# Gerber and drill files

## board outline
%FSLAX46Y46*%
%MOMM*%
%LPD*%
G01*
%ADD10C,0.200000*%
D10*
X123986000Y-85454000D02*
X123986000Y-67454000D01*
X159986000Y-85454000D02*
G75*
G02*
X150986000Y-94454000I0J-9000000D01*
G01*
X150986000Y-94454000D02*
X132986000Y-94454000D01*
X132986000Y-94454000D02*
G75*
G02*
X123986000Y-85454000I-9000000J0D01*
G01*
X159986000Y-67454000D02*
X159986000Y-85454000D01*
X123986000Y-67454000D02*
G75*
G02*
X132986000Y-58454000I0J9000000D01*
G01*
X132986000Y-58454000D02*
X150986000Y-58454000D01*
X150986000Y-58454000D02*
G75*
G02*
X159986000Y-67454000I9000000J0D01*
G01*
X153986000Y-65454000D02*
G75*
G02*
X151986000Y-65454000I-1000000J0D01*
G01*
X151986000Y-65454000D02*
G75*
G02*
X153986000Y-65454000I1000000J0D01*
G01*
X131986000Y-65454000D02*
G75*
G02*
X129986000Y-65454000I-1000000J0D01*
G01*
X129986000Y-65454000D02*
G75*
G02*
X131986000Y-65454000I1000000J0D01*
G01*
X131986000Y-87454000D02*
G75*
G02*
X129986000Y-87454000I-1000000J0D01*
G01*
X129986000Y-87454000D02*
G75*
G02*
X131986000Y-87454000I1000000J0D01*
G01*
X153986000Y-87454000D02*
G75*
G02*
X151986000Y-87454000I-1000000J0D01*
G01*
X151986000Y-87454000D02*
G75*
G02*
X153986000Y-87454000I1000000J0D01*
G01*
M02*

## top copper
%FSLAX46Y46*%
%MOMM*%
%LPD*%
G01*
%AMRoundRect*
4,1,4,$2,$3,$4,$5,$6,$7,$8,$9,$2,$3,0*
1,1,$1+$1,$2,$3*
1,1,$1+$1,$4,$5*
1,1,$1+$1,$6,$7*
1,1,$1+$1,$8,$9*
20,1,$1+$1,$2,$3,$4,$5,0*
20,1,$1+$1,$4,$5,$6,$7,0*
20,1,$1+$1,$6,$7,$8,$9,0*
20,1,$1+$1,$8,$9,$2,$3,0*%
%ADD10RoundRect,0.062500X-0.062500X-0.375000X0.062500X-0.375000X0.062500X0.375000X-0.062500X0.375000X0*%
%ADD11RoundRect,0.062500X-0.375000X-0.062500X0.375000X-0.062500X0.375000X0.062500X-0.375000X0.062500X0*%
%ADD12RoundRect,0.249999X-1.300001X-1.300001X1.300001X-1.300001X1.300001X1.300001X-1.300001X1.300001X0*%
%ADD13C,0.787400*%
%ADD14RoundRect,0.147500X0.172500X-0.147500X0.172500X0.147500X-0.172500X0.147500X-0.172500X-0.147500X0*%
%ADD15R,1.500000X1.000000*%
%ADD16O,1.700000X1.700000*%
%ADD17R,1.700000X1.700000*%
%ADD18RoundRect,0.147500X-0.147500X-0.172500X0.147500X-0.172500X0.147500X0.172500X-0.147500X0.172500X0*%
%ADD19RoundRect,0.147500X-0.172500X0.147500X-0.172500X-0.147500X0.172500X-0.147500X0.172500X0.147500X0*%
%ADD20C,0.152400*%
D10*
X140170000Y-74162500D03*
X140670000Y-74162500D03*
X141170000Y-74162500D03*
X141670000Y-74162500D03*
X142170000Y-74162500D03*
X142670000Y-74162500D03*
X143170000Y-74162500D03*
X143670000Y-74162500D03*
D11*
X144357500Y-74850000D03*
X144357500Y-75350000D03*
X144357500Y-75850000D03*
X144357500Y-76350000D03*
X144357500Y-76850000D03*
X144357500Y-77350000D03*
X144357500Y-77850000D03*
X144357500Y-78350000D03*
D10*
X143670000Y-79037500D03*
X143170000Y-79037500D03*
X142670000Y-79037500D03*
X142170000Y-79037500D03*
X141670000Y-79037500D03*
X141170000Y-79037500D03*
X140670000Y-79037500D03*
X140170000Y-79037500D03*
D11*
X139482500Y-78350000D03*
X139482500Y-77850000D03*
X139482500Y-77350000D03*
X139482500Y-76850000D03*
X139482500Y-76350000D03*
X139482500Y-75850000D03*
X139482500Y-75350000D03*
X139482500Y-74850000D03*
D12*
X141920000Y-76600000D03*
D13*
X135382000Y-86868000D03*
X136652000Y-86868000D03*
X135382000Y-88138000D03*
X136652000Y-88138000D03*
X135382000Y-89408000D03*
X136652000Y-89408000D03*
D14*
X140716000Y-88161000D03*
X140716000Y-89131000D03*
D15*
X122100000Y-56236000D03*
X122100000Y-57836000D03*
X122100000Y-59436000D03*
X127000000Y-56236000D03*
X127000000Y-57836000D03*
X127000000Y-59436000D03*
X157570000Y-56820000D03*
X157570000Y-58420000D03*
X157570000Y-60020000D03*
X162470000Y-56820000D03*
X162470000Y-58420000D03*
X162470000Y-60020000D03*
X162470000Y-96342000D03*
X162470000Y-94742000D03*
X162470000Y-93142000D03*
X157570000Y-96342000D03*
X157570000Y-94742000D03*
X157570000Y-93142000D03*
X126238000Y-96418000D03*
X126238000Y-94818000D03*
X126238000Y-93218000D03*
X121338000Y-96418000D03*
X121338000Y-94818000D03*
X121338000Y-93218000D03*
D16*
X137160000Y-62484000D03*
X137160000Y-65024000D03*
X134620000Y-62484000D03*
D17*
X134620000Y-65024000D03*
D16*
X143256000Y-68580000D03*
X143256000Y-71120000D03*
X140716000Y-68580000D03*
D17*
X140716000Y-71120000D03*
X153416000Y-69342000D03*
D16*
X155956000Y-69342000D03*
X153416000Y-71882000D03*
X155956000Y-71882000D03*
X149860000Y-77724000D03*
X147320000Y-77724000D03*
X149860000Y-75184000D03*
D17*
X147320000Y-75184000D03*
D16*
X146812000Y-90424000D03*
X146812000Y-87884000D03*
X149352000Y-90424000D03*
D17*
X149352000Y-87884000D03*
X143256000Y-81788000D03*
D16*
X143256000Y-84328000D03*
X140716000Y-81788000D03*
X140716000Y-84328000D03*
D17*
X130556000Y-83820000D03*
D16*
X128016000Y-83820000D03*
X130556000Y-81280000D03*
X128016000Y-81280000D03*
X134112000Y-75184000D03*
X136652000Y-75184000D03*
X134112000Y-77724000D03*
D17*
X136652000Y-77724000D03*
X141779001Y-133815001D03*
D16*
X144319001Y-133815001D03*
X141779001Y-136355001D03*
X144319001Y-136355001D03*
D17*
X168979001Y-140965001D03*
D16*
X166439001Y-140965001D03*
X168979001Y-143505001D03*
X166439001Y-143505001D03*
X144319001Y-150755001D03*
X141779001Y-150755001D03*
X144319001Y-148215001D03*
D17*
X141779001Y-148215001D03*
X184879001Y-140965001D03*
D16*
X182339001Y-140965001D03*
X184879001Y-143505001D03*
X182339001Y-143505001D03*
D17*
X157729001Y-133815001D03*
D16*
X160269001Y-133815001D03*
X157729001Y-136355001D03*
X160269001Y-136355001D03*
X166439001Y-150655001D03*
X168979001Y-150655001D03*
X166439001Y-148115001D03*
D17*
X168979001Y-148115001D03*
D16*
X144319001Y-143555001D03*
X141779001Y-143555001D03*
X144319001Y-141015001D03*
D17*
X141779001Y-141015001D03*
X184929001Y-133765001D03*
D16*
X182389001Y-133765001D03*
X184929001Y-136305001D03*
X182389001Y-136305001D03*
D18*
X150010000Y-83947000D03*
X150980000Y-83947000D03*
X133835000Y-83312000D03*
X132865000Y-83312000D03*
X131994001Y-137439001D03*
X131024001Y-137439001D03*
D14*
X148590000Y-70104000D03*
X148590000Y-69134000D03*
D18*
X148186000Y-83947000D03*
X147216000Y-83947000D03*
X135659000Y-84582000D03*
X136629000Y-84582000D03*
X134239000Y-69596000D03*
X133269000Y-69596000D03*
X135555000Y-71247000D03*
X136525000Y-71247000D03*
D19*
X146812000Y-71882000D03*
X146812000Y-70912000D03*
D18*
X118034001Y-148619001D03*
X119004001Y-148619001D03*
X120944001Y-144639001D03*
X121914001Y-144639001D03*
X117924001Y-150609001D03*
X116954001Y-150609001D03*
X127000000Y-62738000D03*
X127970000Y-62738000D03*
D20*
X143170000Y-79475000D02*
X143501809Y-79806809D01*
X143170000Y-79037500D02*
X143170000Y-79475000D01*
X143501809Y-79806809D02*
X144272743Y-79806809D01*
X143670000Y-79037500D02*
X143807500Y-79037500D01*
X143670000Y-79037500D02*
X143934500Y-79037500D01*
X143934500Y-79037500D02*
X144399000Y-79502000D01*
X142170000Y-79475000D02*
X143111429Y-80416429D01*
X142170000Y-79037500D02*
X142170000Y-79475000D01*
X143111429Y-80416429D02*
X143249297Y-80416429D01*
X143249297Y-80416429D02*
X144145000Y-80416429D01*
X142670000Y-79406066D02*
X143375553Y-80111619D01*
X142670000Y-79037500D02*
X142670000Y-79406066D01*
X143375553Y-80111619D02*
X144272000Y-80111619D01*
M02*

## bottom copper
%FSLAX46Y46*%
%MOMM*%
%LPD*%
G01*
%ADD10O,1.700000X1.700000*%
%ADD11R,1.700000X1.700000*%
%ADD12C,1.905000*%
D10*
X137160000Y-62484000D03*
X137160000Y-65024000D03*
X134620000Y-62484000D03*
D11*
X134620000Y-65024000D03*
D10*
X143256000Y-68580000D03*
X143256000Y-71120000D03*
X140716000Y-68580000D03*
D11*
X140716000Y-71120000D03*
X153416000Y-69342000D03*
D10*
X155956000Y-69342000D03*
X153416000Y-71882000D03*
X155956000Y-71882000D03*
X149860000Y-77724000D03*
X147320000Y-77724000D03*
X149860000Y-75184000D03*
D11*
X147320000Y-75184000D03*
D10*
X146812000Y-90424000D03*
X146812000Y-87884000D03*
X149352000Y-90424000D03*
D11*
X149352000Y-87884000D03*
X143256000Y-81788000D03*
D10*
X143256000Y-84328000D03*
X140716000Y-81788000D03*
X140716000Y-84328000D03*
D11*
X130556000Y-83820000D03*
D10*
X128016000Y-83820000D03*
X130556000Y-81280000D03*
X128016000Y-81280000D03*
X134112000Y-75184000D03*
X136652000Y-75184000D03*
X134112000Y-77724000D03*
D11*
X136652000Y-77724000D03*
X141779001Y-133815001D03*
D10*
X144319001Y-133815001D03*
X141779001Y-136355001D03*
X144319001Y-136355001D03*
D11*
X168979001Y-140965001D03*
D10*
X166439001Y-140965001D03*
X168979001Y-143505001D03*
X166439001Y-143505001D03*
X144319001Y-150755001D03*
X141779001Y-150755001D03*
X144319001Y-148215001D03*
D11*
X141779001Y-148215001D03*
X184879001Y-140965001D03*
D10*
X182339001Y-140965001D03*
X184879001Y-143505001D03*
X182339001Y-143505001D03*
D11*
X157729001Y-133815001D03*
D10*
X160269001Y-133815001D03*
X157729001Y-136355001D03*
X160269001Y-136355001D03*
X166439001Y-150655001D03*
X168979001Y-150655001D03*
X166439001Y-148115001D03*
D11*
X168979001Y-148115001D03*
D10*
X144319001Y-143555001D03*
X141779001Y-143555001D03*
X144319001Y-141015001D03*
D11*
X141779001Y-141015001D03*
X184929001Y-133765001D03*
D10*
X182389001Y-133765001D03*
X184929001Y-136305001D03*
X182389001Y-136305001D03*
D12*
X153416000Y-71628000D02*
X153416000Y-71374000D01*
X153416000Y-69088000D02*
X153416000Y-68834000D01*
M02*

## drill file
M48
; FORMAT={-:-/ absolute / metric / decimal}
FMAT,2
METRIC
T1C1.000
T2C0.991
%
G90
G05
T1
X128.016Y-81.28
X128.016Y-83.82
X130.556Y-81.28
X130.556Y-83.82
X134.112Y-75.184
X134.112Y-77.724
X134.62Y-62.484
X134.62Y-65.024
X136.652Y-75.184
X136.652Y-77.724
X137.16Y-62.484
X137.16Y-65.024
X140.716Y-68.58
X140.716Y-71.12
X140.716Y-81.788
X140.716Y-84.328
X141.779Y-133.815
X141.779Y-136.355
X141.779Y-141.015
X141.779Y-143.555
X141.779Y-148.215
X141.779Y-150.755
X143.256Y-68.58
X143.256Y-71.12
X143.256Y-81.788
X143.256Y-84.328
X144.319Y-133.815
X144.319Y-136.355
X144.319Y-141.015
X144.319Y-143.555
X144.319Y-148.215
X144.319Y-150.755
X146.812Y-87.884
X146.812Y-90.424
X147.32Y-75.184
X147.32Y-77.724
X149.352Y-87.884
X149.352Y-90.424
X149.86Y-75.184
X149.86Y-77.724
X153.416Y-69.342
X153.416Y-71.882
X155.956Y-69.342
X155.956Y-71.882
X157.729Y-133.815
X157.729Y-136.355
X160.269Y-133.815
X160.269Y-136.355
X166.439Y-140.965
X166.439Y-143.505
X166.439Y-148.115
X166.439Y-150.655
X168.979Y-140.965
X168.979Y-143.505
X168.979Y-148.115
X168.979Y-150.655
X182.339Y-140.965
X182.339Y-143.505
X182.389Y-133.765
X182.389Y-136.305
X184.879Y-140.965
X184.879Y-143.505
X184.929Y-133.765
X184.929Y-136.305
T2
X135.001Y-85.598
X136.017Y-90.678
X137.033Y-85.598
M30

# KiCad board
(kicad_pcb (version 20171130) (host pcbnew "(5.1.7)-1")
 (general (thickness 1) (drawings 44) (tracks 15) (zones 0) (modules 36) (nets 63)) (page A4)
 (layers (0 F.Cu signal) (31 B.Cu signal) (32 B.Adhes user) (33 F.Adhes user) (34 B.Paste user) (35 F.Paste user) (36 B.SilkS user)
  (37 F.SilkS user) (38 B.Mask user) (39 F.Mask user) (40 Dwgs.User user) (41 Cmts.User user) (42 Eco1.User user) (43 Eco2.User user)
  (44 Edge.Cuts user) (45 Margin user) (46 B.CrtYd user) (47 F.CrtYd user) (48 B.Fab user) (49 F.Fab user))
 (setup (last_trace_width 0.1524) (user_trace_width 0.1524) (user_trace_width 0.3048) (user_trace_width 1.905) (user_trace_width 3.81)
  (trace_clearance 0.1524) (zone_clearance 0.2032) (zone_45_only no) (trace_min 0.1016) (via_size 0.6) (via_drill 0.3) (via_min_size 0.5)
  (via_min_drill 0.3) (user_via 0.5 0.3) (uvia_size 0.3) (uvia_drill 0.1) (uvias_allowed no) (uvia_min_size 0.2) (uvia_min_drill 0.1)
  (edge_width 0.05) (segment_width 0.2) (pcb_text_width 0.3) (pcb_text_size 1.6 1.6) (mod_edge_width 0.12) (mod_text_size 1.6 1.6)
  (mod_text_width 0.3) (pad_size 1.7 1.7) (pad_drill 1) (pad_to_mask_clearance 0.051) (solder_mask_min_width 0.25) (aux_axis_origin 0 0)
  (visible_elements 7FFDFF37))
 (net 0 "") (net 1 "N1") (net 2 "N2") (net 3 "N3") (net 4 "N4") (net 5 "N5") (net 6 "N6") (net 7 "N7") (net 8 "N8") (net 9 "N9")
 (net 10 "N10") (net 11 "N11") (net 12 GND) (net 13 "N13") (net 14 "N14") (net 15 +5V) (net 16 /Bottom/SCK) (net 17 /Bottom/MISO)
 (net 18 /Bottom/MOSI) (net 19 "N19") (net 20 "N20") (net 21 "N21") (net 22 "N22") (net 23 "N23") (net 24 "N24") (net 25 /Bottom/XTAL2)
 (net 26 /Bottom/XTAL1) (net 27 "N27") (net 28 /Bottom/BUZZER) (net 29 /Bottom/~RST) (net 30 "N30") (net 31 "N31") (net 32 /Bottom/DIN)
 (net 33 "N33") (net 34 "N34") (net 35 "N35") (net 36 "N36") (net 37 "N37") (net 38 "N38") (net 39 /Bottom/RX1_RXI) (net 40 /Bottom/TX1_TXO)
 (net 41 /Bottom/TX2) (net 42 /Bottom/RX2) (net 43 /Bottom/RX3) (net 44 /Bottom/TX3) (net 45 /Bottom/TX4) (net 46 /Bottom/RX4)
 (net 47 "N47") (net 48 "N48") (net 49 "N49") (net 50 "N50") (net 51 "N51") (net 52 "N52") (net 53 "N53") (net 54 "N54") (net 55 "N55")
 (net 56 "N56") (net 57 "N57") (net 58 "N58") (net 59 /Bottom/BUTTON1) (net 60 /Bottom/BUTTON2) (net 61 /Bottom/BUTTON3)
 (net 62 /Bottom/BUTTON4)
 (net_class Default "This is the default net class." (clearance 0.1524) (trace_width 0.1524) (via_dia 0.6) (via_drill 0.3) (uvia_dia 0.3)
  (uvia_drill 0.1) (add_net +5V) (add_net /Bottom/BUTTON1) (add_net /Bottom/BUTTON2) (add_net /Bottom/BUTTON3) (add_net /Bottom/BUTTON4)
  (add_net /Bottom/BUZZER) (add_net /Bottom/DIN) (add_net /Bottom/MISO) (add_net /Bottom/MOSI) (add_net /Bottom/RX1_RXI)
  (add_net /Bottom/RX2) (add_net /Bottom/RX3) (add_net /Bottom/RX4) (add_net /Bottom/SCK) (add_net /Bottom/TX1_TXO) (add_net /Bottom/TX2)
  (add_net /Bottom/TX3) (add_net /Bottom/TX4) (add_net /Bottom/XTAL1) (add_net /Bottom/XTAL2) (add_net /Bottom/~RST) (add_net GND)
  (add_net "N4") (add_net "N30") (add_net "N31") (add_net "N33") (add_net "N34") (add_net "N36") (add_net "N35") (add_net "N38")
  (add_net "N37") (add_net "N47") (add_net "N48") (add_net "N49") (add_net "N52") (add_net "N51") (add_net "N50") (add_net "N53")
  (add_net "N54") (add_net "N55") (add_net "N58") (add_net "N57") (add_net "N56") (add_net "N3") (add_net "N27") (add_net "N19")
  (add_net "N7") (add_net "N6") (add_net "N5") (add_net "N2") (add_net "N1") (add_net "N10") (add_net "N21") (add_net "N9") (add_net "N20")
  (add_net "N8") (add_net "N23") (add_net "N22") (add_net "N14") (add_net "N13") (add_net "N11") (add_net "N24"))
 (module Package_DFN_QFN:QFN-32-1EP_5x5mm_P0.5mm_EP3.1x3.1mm (layer F.Cu) (at 141.92 76.6)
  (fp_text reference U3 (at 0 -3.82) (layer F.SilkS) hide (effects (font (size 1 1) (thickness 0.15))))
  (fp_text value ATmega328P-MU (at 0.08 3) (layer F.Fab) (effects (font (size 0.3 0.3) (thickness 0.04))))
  (pad 32 smd roundrect (at -1.75 -2.4375) (size 0.25 0.875) (layers F.Cu F.Paste F.Mask) (roundrect_rratio 0.25) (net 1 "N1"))
  (pad 31 smd roundrect (at -1.25 -2.4375) (size 0.25 0.875) (layers F.Cu F.Paste F.Mask) (roundrect_rratio 0.25) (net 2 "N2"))
  (pad 30 smd roundrect (at -0.75 -2.4375) (size 0.25 0.875) (layers F.Cu F.Paste F.Mask) (roundrect_rratio 0.25) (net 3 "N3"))
  (pad 29 smd roundrect (at -0.25 -2.4375) (size 0.25 0.875) (layers F.Cu F.Paste F.Mask) (roundrect_rratio 0.25) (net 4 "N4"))
  (pad 28 smd roundrect (at 0.25 -2.4375) (size 0.25 0.875) (layers F.Cu F.Paste F.Mask) (roundrect_rratio 0.25) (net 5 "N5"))
  (pad 27 smd roundrect (at 0.75 -2.4375) (size 0.25 0.875) (layers F.Cu F.Paste F.Mask) (roundrect_rratio 0.25) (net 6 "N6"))
  (pad 26 smd roundrect (at 1.25 -2.4375) (size 0.25 0.875) (layers F.Cu F.Paste F.Mask) (roundrect_rratio 0.25) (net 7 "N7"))
  (pad 25 smd roundrect (at 1.75 -2.4375) (size 0.25 0.875) (layers F.Cu F.Paste F.Mask) (roundrect_rratio 0.25) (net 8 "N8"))
  (pad 24 smd roundrect (at 2.4375 -1.75) (size 0.875 0.25) (layers F.Cu F.Paste F.Mask) (roundrect_rratio 0.25) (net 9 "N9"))
  (pad 23 smd roundrect (at 2.4375 -1.25) (size 0.875 0.25) (layers F.Cu F.Paste F.Mask) (roundrect_rratio 0.25) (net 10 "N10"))
  (pad 22 smd roundrect (at 2.4375 -0.75) (size 0.875 0.25) (layers F.Cu F.Paste F.Mask) (roundrect_rratio 0.25) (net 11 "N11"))
  (pad 21 smd roundrect (at 2.4375 -0.25) (size 0.875 0.25) (layers F.Cu F.Paste F.Mask) (roundrect_rratio 0.25) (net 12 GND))
  (pad 20 smd roundrect (at 2.4375 0.25) (size 0.875 0.25) (layers F.Cu F.Paste F.Mask) (roundrect_rratio 0.25) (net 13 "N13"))
  (pad 19 smd roundrect (at 2.4375 0.75) (size 0.875 0.25) (layers F.Cu F.Paste F.Mask) (roundrect_rratio 0.25) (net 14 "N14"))
  (pad 18 smd roundrect (at 2.4375 1.25) (size 0.875 0.25) (layers F.Cu F.Paste F.Mask) (roundrect_rratio 0.25) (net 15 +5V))
  (pad 17 smd roundrect (at 2.4375 1.75) (size 0.875 0.25) (layers F.Cu F.Paste F.Mask) (roundrect_rratio 0.25) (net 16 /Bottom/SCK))
  (pad 16 smd roundrect (at 1.75 2.4375) (size 0.25 0.875) (layers F.Cu F.Paste F.Mask) (roundrect_rratio 0.25) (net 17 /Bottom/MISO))
  (pad 15 smd roundrect (at 1.25 2.4375) (size 0.25 0.875) (layers F.Cu F.Paste F.Mask) (roundrect_rratio 0.25) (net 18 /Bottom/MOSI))
  (pad 14 smd roundrect (at 0.75 2.4375) (size 0.25 0.875) (layers F.Cu F.Paste F.Mask) (roundrect_rratio 0.25) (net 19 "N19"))
  (pad 13 smd roundrect (at 0.25 2.4375) (size 0.25 0.875) (layers F.Cu F.Paste F.Mask) (roundrect_rratio 0.25) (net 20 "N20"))
  (pad 12 smd roundrect (at -0.25 2.4375) (size 0.25 0.875) (layers F.Cu F.Paste F.Mask) (roundrect_rratio 0.25) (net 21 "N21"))
  (pad 11 smd roundrect (at -0.75 2.4375) (size 0.25 0.875) (layers F.Cu F.Paste F.Mask) (roundrect_rratio 0.25) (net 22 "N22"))
  (pad 10 smd roundrect (at -1.25 2.4375) (size 0.25 0.875) (layers F.Cu F.Paste F.Mask) (roundrect_rratio 0.25) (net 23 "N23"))
  (pad 9 smd roundrect (at -1.75 2.4375) (size 0.25 0.875) (layers F.Cu F.Paste F.Mask) (roundrect_rratio 0.25) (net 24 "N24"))
  (pad 8 smd roundrect (at -2.4375 1.75) (size 0.875 0.25) (layers F.Cu F.Paste F.Mask) (roundrect_rratio 0.25) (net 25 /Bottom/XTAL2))
  (pad 7 smd roundrect (at -2.4375 1.25) (size 0.875 0.25) (layers F.Cu F.Paste F.Mask) (roundrect_rratio 0.25) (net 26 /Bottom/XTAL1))
  (pad 6 smd roundrect (at -2.4375 0.75) (size 0.875 0.25) (layers F.Cu F.Paste F.Mask) (roundrect_rratio 0.25) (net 15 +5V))
  (pad 5 smd roundrect (at -2.4375 0.25) (size 0.875 0.25) (layers F.Cu F.Paste F.Mask) (roundrect_rratio 0.25) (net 12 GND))
  (pad 4 smd roundrect (at -2.4375 -0.25) (size 0.875 0.25) (layers F.Cu F.Paste F.Mask) (roundrect_rratio 0.25) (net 15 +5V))
  (pad 3 smd roundrect (at -2.4375 -0.75) (size 0.875 0.25) (layers F.Cu F.Paste F.Mask) (roundrect_rratio 0.25) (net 12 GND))
  (pad 2 smd roundrect (at -2.4375 -1.25) (size 0.875 0.25) (layers F.Cu F.Paste F.Mask) (roundrect_rratio 0.25) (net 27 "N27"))
  (pad 1 smd roundrect (at -2.4375 -1.75) (size 0.875 0.25) (layers F.Cu F.Paste F.Mask) (roundrect_rratio 0.25) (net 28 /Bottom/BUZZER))
  (pad "" smd roundrect (at 1.03 1.03) (size 0.83 0.83) (layers F.Paste) (roundrect_rratio 0.25))
  (pad "" smd roundrect (at 1.03 0) (size 0.83 0.83) (layers F.Paste) (roundrect_rratio 0.25))
  (pad "" smd roundrect (at 1.03 -1.03) (size 0.83 0.83) (layers F.Paste) (roundrect_rratio 0.25))
  (pad "" smd roundrect (at 0 1.03) (size 0.83 0.83) (layers F.Paste) (roundrect_rratio 0.25))
  (pad "" smd roundrect (at 0 0) (size 0.83 0.83) (layers F.Paste) (roundrect_rratio 0.25))
  (pad "" smd roundrect (at 0 -1.03) (size 0.83 0.83) (layers F.Paste) (roundrect_rratio 0.25))
  (pad "" smd roundrect (at -1.03 1.03) (size 0.83 0.83) (layers F.Paste) (roundrect_rratio 0.25))
  (pad "" smd roundrect (at -1.03 0) (size 0.83 0.83) (layers F.Paste) (roundrect_rratio 0.25))
  (pad "" smd roundrect (at -1.03 -1.03) (size 0.83 0.83) (layers F.Paste) (roundrect_rratio 0.25))
  (pad 33 smd roundrect (at 0 0) (size 3.1 3.1) (layers F.Cu F.Mask) (roundrect_rratio 0.08064499999999999) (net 12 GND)))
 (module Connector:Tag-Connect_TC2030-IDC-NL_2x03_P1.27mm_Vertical (layer F.Cu) (at 136.017 88.138 90)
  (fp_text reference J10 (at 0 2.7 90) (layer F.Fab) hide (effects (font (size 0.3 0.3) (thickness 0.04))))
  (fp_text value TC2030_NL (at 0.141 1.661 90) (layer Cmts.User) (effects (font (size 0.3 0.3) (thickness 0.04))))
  (pad 6 connect circle (at 1.27 -0.635 90) (size 0.7874 0.7874) (layers F.Cu F.Mask) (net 15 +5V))
  (pad 5 connect circle (at 1.27 0.635 90) (size 0.7874 0.7874) (layers F.Cu F.Mask) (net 18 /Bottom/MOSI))
  (pad 4 connect circle (at 0 -0.635 90) (size 0.7874 0.7874) (layers F.Cu F.Mask) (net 17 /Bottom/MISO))
  (pad 3 connect circle (at 0 0.635 90) (size 0.7874 0.7874) (layers F.Cu F.Mask) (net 16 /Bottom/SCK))
  (pad 2 connect circle (at -1.27 -0.635 90) (size 0.7874 0.7874) (layers F.Cu F.Mask) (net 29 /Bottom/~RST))
  (pad 1 connect circle (at -1.27 0.635 90) (size 0.7874 0.7874) (layers F.Cu F.Mask) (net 12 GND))
  (pad "" np_thru_hole circle (at -2.54 0 90) (size 0.9906 0.9906) (drill 0.9906) (layers *.Cu *.Mask))
  (pad "" np_thru_hole circle (at 2.54 1.016 90) (size 0.9906 0.9906) (drill 0.9906) (layers *.Cu *.Mask))
  (pad "" np_thru_hole circle (at 2.54 -1.016 90) (size 0.9906 0.9906) (drill 0.9906) (layers *.Cu *.Mask)))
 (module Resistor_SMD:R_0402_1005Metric (layer F.Cu) (at 140.716 88.646 90)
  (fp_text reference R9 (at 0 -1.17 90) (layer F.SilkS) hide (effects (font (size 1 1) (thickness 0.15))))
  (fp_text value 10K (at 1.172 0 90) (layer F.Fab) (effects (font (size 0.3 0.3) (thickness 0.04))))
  (pad 2 smd roundrect (at 0.485 0 90) (size 0.59 0.64) (layers F.Cu F.Paste F.Mask) (roundrect_rratio 0.25) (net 4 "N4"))
  (pad 1 smd roundrect (at -0.485 0 90) (size 0.59 0.64) (layers F.Cu F.Paste F.Mask) (roundrect_rratio 0.25) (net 15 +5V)))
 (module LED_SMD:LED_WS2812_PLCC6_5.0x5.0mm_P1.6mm (layer F.Cu) (at 124.55 57.836)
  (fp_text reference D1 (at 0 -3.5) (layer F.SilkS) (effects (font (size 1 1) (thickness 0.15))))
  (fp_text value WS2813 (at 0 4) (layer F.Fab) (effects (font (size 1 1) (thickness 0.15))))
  (pad 1 smd rect (at -2.45 -1.6) (size 1.5 1) (layers F.Cu F.Paste F.Mask) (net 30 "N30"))
  (pad 2 smd rect (at -2.45 0) (size 1.5 1) (layers F.Cu F.Paste F.Mask) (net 15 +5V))
  (pad 3 smd rect (at -2.45 1.6) (size 1.5 1) (layers F.Cu F.Paste F.Mask) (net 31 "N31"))
  (pad 6 smd rect (at 2.45 -1.6) (size 1.5 1) (layers F.Cu F.Paste F.Mask) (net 12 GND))
  (pad 5 smd rect (at 2.45 0) (size 1.5 1) (layers F.Cu F.Paste F.Mask) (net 12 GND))
  (pad 4 smd rect (at 2.45 1.6) (size 1.5 1) (layers F.Cu F.Paste F.Mask) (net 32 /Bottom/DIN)))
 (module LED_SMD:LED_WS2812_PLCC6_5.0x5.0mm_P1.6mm (layer F.Cu) (at 160.02 58.42)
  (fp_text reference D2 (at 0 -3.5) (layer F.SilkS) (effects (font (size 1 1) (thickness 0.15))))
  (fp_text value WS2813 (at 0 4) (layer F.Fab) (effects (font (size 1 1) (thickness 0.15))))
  (pad 1 smd rect (at -2.45 -1.6) (size 1.5 1) (layers F.Cu F.Paste F.Mask) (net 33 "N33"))
  (pad 2 smd rect (at -2.45 0) (size 1.5 1) (layers F.Cu F.Paste F.Mask) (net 15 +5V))
  (pad 3 smd rect (at -2.45 1.6) (size 1.5 1) (layers F.Cu F.Paste F.Mask) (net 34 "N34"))
  (pad 6 smd rect (at 2.45 -1.6) (size 1.5 1) (layers F.Cu F.Paste F.Mask) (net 32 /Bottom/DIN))
  (pad 5 smd rect (at 2.45 0) (size 1.5 1) (layers F.Cu F.Paste F.Mask) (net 12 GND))
  (pad 4 smd rect (at 2.45 1.6) (size 1.5 1) (layers F.Cu F.Paste F.Mask) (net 31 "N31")))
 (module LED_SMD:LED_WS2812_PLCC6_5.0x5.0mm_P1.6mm (layer F.Cu) (at 160.02 94.742)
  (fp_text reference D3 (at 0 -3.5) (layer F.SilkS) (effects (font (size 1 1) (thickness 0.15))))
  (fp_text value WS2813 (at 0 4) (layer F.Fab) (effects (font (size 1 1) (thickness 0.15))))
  (pad 4 smd rect (at 2.45 1.6) (size 1.5 1) (layers F.Cu F.Paste F.Mask) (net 34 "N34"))
  (pad 5 smd rect (at 2.45 0) (size 1.5 1) (layers F.Cu F.Paste F.Mask) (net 12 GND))
  (pad 6 smd rect (at 2.45 -1.6) (size 1.5 1) (layers F.Cu F.Paste F.Mask) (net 31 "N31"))
  (pad 3 smd rect (at -2.45 1.6) (size 1.5 1) (layers F.Cu F.Paste F.Mask) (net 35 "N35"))
  (pad 2 smd rect (at -2.45 0) (size 1.5 1) (layers F.Cu F.Paste F.Mask) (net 15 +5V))
  (pad 1 smd rect (at -2.45 -1.6) (size 1.5 1) (layers F.Cu F.Paste F.Mask) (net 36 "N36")))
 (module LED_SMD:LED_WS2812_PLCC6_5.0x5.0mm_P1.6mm (layer F.Cu) (at 123.788 94.818)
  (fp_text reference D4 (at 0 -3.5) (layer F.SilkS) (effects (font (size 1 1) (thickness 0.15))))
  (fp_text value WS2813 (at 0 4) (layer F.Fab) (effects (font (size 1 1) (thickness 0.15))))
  (pad 4 smd rect (at 2.45 1.6) (size 1.5 1) (layers F.Cu F.Paste F.Mask) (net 35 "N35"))
  (pad 5 smd rect (at 2.45 0) (size 1.5 1) (layers F.Cu F.Paste F.Mask) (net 12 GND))
  (pad 6 smd rect (at 2.45 -1.6) (size 1.5 1) (layers F.Cu F.Paste F.Mask) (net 34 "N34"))
  (pad 3 smd rect (at -2.45 1.6) (size 1.5 1) (layers F.Cu F.Paste F.Mask) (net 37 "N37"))
  (pad 2 smd rect (at -2.45 0) (size 1.5 1) (layers F.Cu F.Paste F.Mask) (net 15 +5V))
  (pad 1 smd rect (at -2.45 -1.6) (size 1.5 1) (layers F.Cu F.Paste F.Mask) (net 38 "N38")))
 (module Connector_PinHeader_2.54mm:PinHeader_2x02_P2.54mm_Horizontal (layer F.Cu) (at 134.62 65.024 90)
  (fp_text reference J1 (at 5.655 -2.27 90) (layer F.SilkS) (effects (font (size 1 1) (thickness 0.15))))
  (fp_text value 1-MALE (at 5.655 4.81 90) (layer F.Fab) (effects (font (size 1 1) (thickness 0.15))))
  (pad 4 thru_hole oval (at 2.54 2.54 90) (size 1.7 1.7) (drill 1) (layers *.Cu *.Mask) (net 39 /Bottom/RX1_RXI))
  (pad 3 thru_hole oval (at 0 2.54 90) (size 1.7 1.7) (drill 1) (layers *.Cu *.Mask) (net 12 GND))
  (pad 2 thru_hole oval (at 2.54 0 90) (size 1.7 1.7) (drill 1) (layers *.Cu *.Mask) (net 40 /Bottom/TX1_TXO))
  (pad 1 thru_hole rect (at 0 0 90) (size 1.7 1.7) (drill 1) (layers *.Cu *.Mask) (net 15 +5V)))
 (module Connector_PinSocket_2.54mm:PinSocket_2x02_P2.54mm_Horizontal (layer B.Cu) (at 140.716 71.12 270)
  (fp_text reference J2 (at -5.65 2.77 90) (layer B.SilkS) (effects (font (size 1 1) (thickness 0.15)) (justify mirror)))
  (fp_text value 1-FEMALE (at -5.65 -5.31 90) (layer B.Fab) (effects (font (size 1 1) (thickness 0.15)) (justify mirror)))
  (pad 4 thru_hole oval (at -2.54 -2.54 270) (size 1.7 1.7) (drill 1) (layers *.Cu *.Mask) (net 39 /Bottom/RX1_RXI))
  (pad 3 thru_hole oval (at 0 -2.54 270) (size 1.7 1.7) (drill 1) (layers *.Cu *.Mask) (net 12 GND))
  (pad 2 thru_hole oval (at -2.54 0 270) (size 1.7 1.7) (drill 1) (layers *.Cu *.Mask) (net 40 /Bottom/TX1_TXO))
  (pad 1 thru_hole rect (at 0 0 270) (size 1.7 1.7) (drill 1) (layers *.Cu *.Mask) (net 15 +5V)))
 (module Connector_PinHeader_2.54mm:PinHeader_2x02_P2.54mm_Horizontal (layer F.Cu) (at 153.416 69.342)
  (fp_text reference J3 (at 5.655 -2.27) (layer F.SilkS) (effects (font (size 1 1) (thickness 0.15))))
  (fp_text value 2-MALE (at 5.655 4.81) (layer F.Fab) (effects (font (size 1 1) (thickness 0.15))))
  (pad 1 thru_hole rect (at 0 0) (size 1.7 1.7) (drill 1) (layers *.Cu *.Mask) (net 15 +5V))
  (pad 2 thru_hole oval (at 2.54 0) (size 1.7 1.7) (drill 1) (layers *.Cu *.Mask) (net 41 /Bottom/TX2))
  (pad 3 thru_hole oval (at 0 2.54) (size 1.7 1.7) (drill 1) (layers *.Cu *.Mask) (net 12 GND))
  (pad 4 thru_hole oval (at 2.54 2.54) (size 1.7 1.7) (drill 1) (layers *.Cu *.Mask) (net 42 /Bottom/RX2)))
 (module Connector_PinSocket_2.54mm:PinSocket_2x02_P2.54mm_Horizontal (layer B.Cu) (at 147.32 75.184 180)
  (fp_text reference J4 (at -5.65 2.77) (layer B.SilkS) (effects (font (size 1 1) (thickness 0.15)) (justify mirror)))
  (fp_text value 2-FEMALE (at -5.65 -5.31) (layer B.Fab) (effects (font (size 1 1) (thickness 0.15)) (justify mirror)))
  (pad 4 thru_hole oval (at -2.54 -2.54 180) (size 1.7 1.7) (drill 1) (layers *.Cu *.Mask) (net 42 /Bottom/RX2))
  (pad 3 thru_hole oval (at 0 -2.54 180) (size 1.7 1.7) (drill 1) (layers *.Cu *.Mask) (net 12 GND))
  (pad 2 thru_hole oval (at -2.54 0 180) (size 1.7 1.7) (drill 1) (layers *.Cu *.Mask) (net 41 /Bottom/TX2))
  (pad 1 thru_hole rect (at 0 0 180) (size 1.7 1.7) (drill 1) (layers *.Cu *.Mask) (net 15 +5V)))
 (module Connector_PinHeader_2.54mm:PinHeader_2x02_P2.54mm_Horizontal (layer F.Cu) (at 149.352 87.884 270)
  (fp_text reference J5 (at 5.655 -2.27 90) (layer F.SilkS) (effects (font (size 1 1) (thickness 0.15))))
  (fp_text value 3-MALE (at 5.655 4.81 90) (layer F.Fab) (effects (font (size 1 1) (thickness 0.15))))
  (pad 4 thru_hole oval (at 2.54 2.54 270) (size 1.7 1.7) (drill 1) (layers *.Cu *.Mask) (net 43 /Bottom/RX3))
  (pad 3 thru_hole oval (at 0 2.54 270) (size 1.7 1.7) (drill 1) (layers *.Cu *.Mask) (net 12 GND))
  (pad 2 thru_hole oval (at 2.54 0 270) (size 1.7 1.7) (drill 1) (layers *.Cu *.Mask) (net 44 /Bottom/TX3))
  (pad 1 thru_hole rect (at 0 0 270) (size 1.7 1.7) (drill 1) (layers *.Cu *.Mask) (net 15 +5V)))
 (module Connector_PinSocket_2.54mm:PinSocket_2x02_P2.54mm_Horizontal (layer B.Cu) (at 143.256 81.788 90)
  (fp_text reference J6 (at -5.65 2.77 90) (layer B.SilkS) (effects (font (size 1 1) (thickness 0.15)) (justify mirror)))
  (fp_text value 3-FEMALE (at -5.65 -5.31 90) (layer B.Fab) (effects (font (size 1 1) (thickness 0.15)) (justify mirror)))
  (pad 1 thru_hole rect (at 0 0 90) (size 1.7 1.7) (drill 1) (layers *.Cu *.Mask) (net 15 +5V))
  (pad 2 thru_hole oval (at -2.54 0 90) (size 1.7 1.7) (drill 1) (layers *.Cu *.Mask) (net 44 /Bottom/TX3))
  (pad 3 thru_hole oval (at 0 -2.54 90) (size 1.7 1.7) (drill 1) (layers *.Cu *.Mask) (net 12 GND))
  (pad 4 thru_hole oval (at -2.54 -2.54 90) (size 1.7 1.7) (drill 1) (layers *.Cu *.Mask) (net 43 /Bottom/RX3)))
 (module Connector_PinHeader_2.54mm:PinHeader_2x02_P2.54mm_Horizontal (layer F.Cu) (at 130.556 83.82 180)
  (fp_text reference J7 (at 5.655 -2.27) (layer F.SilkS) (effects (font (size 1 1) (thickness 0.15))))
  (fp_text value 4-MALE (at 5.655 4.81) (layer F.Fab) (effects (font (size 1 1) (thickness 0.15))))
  (pad 1 thru_hole rect (at 0 0 180) (size 1.7 1.7) (drill 1) (layers *.Cu *.Mask) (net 15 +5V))
  (pad 2 thru_hole oval (at 2.54 0 180) (size 1.7 1.7) (drill 1) (layers *.Cu *.Mask) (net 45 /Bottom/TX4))
  (pad 3 thru_hole oval (at 0 2.54 180) (size 1.7 1.7) (drill 1) (layers *.Cu *.Mask) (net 12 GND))
  (pad 4 thru_hole oval (at 2.54 2.54 180) (size 1.7 1.7) (drill 1) (layers *.Cu *.Mask) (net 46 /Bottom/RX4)))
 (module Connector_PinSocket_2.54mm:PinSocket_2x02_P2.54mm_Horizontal (layer B.Cu) (at 136.652 77.724)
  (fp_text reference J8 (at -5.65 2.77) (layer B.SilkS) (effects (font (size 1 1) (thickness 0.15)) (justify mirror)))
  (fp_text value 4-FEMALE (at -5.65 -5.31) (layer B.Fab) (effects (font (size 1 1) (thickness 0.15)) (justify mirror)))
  (pad 4 thru_hole oval (at -2.54 -2.54) (size 1.7 1.7) (drill 1) (layers *.Cu *.Mask) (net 46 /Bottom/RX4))
  (pad 3 thru_hole oval (at 0 -2.54) (size 1.7 1.7) (drill 1) (layers *.Cu *.Mask) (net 12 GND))
  (pad 2 thru_hole oval (at -2.54 0) (size 1.7 1.7) (drill 1) (layers *.Cu *.Mask) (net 45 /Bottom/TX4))
  (pad 1 thru_hole rect (at 0 0) (size 1.7 1.7) (drill 1) (layers *.Cu *.Mask) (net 15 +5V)))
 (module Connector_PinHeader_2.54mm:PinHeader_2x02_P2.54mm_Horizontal (layer F.Cu) (at 141.779001 133.815001)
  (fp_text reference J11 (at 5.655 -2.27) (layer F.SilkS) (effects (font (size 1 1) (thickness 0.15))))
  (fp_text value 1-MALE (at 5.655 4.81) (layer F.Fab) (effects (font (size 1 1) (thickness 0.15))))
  (pad 1 thru_hole rect (at 0 0) (size 1.7 1.7) (drill 1) (layers *.Cu *.Mask) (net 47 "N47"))
  (pad 2 thru_hole oval (at 2.54 0) (size 1.7 1.7) (drill 1) (layers *.Cu *.Mask) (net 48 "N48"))
  (pad 3 thru_hole oval (at 0 2.54) (size 1.7 1.7) (drill 1) (layers *.Cu *.Mask) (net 12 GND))
  (pad 4 thru_hole oval (at 2.54 2.54) (size 1.7 1.7) (drill 1) (layers *.Cu *.Mask) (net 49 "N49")))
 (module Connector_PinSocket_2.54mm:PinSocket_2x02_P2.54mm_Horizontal (layer F.Cu) (at 168.979001 140.965001)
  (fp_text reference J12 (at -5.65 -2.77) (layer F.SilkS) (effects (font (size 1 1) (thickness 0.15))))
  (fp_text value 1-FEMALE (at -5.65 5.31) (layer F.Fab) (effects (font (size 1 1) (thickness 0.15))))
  (pad 1 thru_hole rect (at 0 0) (size 1.7 1.7) (drill 1) (layers *.Cu *.Mask) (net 47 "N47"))
  (pad 2 thru_hole oval (at -2.54 0) (size 1.7 1.7) (drill 1) (layers *.Cu *.Mask) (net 48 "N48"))
  (pad 3 thru_hole oval (at 0 2.54) (size 1.7 1.7) (drill 1) (layers *.Cu *.Mask) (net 12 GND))
  (pad 4 thru_hole oval (at -2.54 2.54) (size 1.7 1.7) (drill 1) (layers *.Cu *.Mask) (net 49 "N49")))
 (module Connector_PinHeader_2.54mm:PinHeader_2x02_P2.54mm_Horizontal (layer F.Cu) (at 141.779001 148.215001)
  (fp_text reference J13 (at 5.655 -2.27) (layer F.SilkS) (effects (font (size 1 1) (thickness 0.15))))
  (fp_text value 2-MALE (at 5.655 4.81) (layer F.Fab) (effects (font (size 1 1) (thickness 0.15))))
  (pad 4 thru_hole oval (at 2.54 2.54) (size 1.7 1.7) (drill 1) (layers *.Cu *.Mask) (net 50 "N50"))
  (pad 3 thru_hole oval (at 0 2.54) (size 1.7 1.7) (drill 1) (layers *.Cu *.Mask) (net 12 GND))
  (pad 2 thru_hole oval (at 2.54 0) (size 1.7 1.7) (drill 1) (layers *.Cu *.Mask) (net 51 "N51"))
  (pad 1 thru_hole rect (at 0 0) (size 1.7 1.7) (drill 1) (layers *.Cu *.Mask) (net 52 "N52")))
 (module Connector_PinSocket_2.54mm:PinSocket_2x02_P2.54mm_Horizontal (layer F.Cu) (at 184.879001 140.965001)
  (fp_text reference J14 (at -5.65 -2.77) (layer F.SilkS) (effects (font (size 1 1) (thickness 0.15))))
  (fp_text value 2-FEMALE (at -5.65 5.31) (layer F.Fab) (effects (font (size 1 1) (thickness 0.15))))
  (pad 1 thru_hole rect (at 0 0) (size 1.7 1.7) (drill 1) (layers *.Cu *.Mask) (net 52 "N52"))
  (pad 2 thru_hole oval (at -2.54 0) (size 1.7 1.7) (drill 1) (layers *.Cu *.Mask) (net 51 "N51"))
  (pad 3 thru_hole oval (at 0 2.54) (size 1.7 1.7) (drill 1) (layers *.Cu *.Mask) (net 12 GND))
  (pad 4 thru_hole oval (at -2.54 2.54) (size 1.7 1.7) (drill 1) (layers *.Cu *.Mask) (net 50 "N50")))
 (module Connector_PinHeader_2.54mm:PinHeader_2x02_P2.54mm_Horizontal (layer F.Cu) (at 157.729001 133.815001)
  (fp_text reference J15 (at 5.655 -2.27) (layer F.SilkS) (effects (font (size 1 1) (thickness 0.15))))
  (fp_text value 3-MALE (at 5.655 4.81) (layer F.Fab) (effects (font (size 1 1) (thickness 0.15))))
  (pad 1 thru_hole rect (at 0 0) (size 1.7 1.7) (drill 1) (layers *.Cu *.Mask) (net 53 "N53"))
  (pad 2 thru_hole oval (at 2.54 0) (size 1.7 1.7) (drill 1) (layers *.Cu *.Mask) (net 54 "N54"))
  (pad 3 thru_hole oval (at 0 2.54) (size 1.7 1.7) (drill 1) (layers *.Cu *.Mask) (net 12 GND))
  (pad 4 thru_hole oval (at 2.54 2.54) (size 1.7 1.7) (drill 1) (layers *.Cu *.Mask) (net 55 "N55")))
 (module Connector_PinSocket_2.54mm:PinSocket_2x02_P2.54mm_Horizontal (layer F.Cu) (at 168.979001 148.115001)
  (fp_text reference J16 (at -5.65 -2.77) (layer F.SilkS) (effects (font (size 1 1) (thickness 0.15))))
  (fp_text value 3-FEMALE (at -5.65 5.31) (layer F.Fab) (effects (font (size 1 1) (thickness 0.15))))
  (pad 4 thru_hole oval (at -2.54 2.54) (size 1.7 1.7) (drill 1) (layers *.Cu *.Mask) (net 55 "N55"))
  (pad 3 thru_hole oval (at 0 2.54) (size 1.7 1.7) (drill 1) (layers *.Cu *.Mask) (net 12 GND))
  (pad 2 thru_hole oval (at -2.54 0) (size 1.7 1.7) (drill 1) (layers *.Cu *.Mask) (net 54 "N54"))
  (pad 1 thru_hole rect (at 0 0) (size 1.7 1.7) (drill 1) (layers *.Cu *.Mask) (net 53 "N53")))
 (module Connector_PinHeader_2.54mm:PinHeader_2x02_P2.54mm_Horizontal (layer F.Cu) (at 141.779001 141.015001)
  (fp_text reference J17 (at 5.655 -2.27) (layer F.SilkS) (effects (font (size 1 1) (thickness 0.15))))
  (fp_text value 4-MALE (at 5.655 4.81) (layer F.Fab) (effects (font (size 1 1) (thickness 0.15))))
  (pad 4 thru_hole oval (at 2.54 2.54) (size 1.7 1.7) (drill 1) (layers *.Cu *.Mask) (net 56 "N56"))
  (pad 3 thru_hole oval (at 0 2.54) (size 1.7 1.7) (drill 1) (layers *.Cu *.Mask) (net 12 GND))
  (pad 2 thru_hole oval (at 2.54 0) (size 1.7 1.7) (drill 1) (layers *.Cu *.Mask) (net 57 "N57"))
  (pad 1 thru_hole rect (at 0 0) (size 1.7 1.7) (drill 1) (layers *.Cu *.Mask) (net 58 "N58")))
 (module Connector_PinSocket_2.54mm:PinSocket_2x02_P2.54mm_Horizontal (layer F.Cu) (at 184.929001 133.765001)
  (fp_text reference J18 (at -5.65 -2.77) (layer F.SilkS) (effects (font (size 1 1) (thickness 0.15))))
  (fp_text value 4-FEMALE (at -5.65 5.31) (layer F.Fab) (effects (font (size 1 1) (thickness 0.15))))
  (pad 1 thru_hole rect (at 0 0) (size 1.7 1.7) (drill 1) (layers *.Cu *.Mask) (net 58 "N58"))
  (pad 2 thru_hole oval (at -2.54 0) (size 1.7 1.7) (drill 1) (layers *.Cu *.Mask) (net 57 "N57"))
  (pad 3 thru_hole oval (at 0 2.54) (size 1.7 1.7) (drill 1) (layers *.Cu *.Mask) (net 12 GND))
  (pad 4 thru_hole oval (at -2.54 2.54) (size 1.7 1.7) (drill 1) (layers *.Cu *.Mask) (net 56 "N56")))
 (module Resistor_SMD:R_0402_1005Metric (layer F.Cu) (at 150.495 83.947)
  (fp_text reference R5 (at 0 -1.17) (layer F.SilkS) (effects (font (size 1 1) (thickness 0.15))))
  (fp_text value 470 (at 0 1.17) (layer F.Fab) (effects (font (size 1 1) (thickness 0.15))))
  (pad 1 smd roundrect (at -0.485 0) (size 0.59 0.64) (layers F.Cu F.Paste F.Mask) (roundrect_rratio 0.25) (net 43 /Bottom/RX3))
  (pad 2 smd roundrect (at 0.485 0) (size 0.59 0.64) (layers F.Cu F.Paste F.Mask) (roundrect_rratio 0.25) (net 21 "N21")))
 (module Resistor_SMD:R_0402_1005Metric (layer F.Cu) (at 133.35 83.312)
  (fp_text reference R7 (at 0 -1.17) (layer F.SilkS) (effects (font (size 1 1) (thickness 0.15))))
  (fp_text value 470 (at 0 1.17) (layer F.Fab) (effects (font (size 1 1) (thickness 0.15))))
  (pad 2 smd roundrect (at 0.485 0) (size 0.59 0.64) (layers F.Cu F.Paste F.Mask) (roundrect_rratio 0.25) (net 20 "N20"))
  (pad 1 smd roundrect (at -0.485 0) (size 0.59 0.64) (layers F.Cu F.Paste F.Mask) (roundrect_rratio 0.25) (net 46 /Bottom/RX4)))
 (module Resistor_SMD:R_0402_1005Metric (layer F.Cu) (at 131.509001 137.439001)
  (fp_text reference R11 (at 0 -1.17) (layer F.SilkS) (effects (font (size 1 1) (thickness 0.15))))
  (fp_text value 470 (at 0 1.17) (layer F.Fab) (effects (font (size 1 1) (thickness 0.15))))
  (pad 2 smd roundrect (at 0.485 0) (size 0.59 0.64) (layers F.Cu F.Paste F.Mask) (roundrect_rratio 0.25) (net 19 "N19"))
  (pad 1 smd roundrect (at -0.485 0) (size 0.59 0.64) (layers F.Cu F.Paste F.Mask) (roundrect_rratio 0.25) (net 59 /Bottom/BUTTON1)))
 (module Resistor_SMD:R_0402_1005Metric (layer F.Cu) (at 148.59 69.619 90)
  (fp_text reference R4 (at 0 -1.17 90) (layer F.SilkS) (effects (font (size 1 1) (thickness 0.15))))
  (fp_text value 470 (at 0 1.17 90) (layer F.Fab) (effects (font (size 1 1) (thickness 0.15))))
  (pad 1 smd roundrect (at -0.485 0 90) (size 0.59 0.64) (layers F.Cu F.Paste F.Mask) (roundrect_rratio 0.25) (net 41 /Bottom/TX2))
  (pad 2 smd roundrect (at 0.485 0 90) (size 0.59 0.64) (layers F.Cu F.Paste F.Mask) (roundrect_rratio 0.25) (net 10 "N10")))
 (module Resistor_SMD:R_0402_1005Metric (layer F.Cu) (at 147.701 83.947)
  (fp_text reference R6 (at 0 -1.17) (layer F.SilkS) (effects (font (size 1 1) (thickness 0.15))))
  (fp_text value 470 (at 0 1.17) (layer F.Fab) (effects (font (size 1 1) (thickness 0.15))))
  (pad 2 smd roundrect (at 0.485 0) (size 0.59 0.64) (layers F.Cu F.Paste F.Mask) (roundrect_rratio 0.25) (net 9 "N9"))
  (pad 1 smd roundrect (at -0.485 0) (size 0.59 0.64) (layers F.Cu F.Paste F.Mask) (roundrect_rratio 0.25) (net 44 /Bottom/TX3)))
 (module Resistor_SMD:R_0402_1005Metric (layer F.Cu) (at 136.144 84.582)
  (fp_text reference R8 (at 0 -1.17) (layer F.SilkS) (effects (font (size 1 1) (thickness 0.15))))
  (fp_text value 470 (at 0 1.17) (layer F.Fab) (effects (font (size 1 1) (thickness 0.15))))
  (pad 1 smd roundrect (at -0.485 0) (size 0.59 0.64) (layers F.Cu F.Paste F.Mask) (roundrect_rratio 0.25) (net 45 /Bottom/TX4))
  (pad 2 smd roundrect (at 0.485 0) (size 0.59 0.64) (layers F.Cu F.Paste F.Mask) (roundrect_rratio 0.25) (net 8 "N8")))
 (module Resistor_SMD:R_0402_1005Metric (layer F.Cu) (at 133.754 69.596)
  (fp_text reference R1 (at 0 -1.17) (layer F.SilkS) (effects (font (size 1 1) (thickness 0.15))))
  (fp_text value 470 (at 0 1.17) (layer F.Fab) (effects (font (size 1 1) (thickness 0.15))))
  (pad 2 smd roundrect (at 0.485 0) (size 0.59 0.64) (layers F.Cu F.Paste F.Mask) (roundrect_rratio 0.25) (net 3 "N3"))
  (pad 1 smd roundrect (at -0.485 0) (size 0.59 0.64) (layers F.Cu F.Paste F.Mask) (roundrect_rratio 0.25) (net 39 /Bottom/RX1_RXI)))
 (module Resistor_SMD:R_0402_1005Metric (layer F.Cu) (at 136.04 71.247)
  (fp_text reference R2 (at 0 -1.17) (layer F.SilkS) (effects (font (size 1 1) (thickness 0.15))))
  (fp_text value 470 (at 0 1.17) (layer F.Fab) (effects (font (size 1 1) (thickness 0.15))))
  (pad 1 smd roundrect (at -0.485 0) (size 0.59 0.64) (layers F.Cu F.Paste F.Mask) (roundrect_rratio 0.25) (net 40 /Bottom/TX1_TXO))
  (pad 2 smd roundrect (at 0.485 0) (size 0.59 0.64) (layers F.Cu F.Paste F.Mask) (roundrect_rratio 0.25) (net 2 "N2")))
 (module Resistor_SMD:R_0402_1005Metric (layer F.Cu) (at 146.812 71.397 270)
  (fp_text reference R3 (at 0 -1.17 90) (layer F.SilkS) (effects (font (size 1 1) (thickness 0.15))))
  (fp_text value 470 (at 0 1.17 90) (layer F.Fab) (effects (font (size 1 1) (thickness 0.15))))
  (pad 2 smd roundrect (at 0.485 0 270) (size 0.59 0.64) (layers F.Cu F.Paste F.Mask) (roundrect_rratio 0.25) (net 1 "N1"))
  (pad 1 smd roundrect (at -0.485 0 270) (size 0.59 0.64) (layers F.Cu F.Paste F.Mask) (roundrect_rratio 0.25) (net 42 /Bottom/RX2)))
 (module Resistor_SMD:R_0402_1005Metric (layer F.Cu) (at 118.519001 148.619001)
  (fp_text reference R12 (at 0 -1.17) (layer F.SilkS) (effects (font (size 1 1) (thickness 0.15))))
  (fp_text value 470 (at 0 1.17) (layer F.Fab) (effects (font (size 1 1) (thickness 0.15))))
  (pad 1 smd roundrect (at -0.485 0) (size 0.59 0.64) (layers F.Cu F.Paste F.Mask) (roundrect_rratio 0.25) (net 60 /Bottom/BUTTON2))
  (pad 2 smd roundrect (at 0.485 0) (size 0.59 0.64) (layers F.Cu F.Paste F.Mask) (roundrect_rratio 0.25) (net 7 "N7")))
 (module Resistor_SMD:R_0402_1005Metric (layer F.Cu) (at 121.429001 144.639001)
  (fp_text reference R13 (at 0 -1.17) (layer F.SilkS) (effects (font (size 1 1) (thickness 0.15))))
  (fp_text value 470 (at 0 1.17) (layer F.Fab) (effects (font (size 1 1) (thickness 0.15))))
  (pad 1 smd roundrect (at -0.485 0) (size 0.59 0.64) (layers F.Cu F.Paste F.Mask) (roundrect_rratio 0.25) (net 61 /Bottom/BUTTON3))
  (pad 2 smd roundrect (at 0.485 0) (size 0.59 0.64) (layers F.Cu F.Paste F.Mask) (roundrect_rratio 0.25) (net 6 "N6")))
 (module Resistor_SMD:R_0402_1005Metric (layer F.Cu) (at 117.439001 150.609001)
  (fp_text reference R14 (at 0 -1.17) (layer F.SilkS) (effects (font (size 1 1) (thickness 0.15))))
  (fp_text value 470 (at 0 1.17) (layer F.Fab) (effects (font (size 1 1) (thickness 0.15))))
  (pad 2 smd roundrect (at 0.485 0) (size 0.59 0.64) (layers F.Cu F.Paste F.Mask) (roundrect_rratio 0.25) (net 5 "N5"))
  (pad 1 smd roundrect (at -0.485 0) (size 0.59 0.64) (layers F.Cu F.Paste F.Mask) (roundrect_rratio 0.25) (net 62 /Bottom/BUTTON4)))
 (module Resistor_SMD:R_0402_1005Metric (layer F.Cu) (at 127.485 62.738)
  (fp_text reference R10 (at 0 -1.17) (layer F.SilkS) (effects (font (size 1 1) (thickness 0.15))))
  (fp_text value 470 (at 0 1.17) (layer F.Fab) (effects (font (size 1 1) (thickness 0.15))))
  (pad 1 smd roundrect (at -0.485 0) (size 0.59 0.64) (layers F.Cu F.Paste F.Mask) (roundrect_rratio 0.25) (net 32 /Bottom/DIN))
  (pad 2 smd roundrect (at 0.485 0) (size 0.59 0.64) (layers F.Cu F.Paste F.Mask) (roundrect_rratio 0.25) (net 27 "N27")))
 (gr_line (start 123.986 85.454) (end 123.986 67.454) (layer Edge.Cuts) (width 0.2))
 (gr_arc (start 159.986 94.454) (end 150.986 94.454) (angle -270) (layer Edge.Cuts) (width 0.2))
 (gr_line (start 150.986 94.454) (end 132.986 94.454) (layer Edge.Cuts) (width 0.2))
 (gr_arc (start 123.986 94.454) (end 123.986 85.454) (angle -270) (layer Edge.Cuts) (width 0.2))
 (gr_line (start 159.986 67.454) (end 159.986 85.454) (layer Edge.Cuts) (width 0.2))
 (gr_arc (start 123.986 58.454) (end 132.986 58.454) (angle -270) (layer Edge.Cuts) (width 0.2))
 (gr_line (start 132.986 58.454) (end 150.986 58.454) (layer Edge.Cuts) (width 0.2))
 (gr_arc (start 159.986 58.454) (end 159.986 67.454) (angle -270) (layer Edge.Cuts) (width 0.2))
 (gr_circle (center 152.986 65.454) (end 153.986 65.454) (layer Edge.Cuts) (width 0.2))
 (gr_circle (center 130.986 65.454) (end 131.986 65.454) (layer Edge.Cuts) (width 0.2))
 (gr_circle (center 130.986 87.454) (end 131.986 87.454) (layer Edge.Cuts) (width 0.2))
 (gr_circle (center 152.986 87.454) (end 153.986 87.454) (layer Edge.Cuts) (width 0.2))
 (segment (start 153.416 71.628) (end 153.416 71.374) (width 1.905) (layer B.Cu) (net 12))
 (segment (start 153.416 69.088) (end 153.416 68.834) (width 1.905) (layer B.Cu) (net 15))
 (segment (start 143.17 79.475) (end 143.501809 79.806809) (width 0.1524) (layer F.Cu) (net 18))
 (segment (start 143.17 79.0375) (end 143.17 79.475) (width 0.1524) (layer F.Cu) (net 18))
 (segment (start 143.501809 79.806809) (end 144.272743 79.806809) (width 0.1524) (layer F.Cu) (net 18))
 (segment (start 143.67 79.0375) (end 143.8075 79.0375) (width 0.1524) (layer F.Cu) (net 17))
 (segment (start 143.67 79.0375) (end 143.9345 79.0375) (width 0.1524) (layer F.Cu) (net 17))
 (segment (start 143.9345 79.0375) (end 144.399 79.502) (width 0.1524) (layer F.Cu) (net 17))
 (segment (start 142.17 79.475) (end 143.111429 80.416429) (width 0.1524) (layer F.Cu) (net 20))
 (segment (start 142.17 79.0375) (end 142.17 79.475) (width 0.1524) (layer F.Cu) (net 20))
 (segment (start 143.111429 80.416429) (end 143.249297 80.416429) (width 0.1524) (layer F.Cu) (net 20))
 (segment (start 143.249297 80.416429) (end 144.145 80.416429) (width 0.1524) (layer F.Cu) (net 20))
 (segment (start 142.67 79.406066) (end 143.375553 80.111619) (width 0.1524) (layer F.Cu) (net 19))
 (segment (start 142.67 79.0375) (end 142.67 79.406066) (width 0.1524) (layer F.Cu) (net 19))
 (segment (start 143.375553 80.111619) (end 144.272 80.111619) (width 0.1524) (layer F.Cu) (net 19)))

